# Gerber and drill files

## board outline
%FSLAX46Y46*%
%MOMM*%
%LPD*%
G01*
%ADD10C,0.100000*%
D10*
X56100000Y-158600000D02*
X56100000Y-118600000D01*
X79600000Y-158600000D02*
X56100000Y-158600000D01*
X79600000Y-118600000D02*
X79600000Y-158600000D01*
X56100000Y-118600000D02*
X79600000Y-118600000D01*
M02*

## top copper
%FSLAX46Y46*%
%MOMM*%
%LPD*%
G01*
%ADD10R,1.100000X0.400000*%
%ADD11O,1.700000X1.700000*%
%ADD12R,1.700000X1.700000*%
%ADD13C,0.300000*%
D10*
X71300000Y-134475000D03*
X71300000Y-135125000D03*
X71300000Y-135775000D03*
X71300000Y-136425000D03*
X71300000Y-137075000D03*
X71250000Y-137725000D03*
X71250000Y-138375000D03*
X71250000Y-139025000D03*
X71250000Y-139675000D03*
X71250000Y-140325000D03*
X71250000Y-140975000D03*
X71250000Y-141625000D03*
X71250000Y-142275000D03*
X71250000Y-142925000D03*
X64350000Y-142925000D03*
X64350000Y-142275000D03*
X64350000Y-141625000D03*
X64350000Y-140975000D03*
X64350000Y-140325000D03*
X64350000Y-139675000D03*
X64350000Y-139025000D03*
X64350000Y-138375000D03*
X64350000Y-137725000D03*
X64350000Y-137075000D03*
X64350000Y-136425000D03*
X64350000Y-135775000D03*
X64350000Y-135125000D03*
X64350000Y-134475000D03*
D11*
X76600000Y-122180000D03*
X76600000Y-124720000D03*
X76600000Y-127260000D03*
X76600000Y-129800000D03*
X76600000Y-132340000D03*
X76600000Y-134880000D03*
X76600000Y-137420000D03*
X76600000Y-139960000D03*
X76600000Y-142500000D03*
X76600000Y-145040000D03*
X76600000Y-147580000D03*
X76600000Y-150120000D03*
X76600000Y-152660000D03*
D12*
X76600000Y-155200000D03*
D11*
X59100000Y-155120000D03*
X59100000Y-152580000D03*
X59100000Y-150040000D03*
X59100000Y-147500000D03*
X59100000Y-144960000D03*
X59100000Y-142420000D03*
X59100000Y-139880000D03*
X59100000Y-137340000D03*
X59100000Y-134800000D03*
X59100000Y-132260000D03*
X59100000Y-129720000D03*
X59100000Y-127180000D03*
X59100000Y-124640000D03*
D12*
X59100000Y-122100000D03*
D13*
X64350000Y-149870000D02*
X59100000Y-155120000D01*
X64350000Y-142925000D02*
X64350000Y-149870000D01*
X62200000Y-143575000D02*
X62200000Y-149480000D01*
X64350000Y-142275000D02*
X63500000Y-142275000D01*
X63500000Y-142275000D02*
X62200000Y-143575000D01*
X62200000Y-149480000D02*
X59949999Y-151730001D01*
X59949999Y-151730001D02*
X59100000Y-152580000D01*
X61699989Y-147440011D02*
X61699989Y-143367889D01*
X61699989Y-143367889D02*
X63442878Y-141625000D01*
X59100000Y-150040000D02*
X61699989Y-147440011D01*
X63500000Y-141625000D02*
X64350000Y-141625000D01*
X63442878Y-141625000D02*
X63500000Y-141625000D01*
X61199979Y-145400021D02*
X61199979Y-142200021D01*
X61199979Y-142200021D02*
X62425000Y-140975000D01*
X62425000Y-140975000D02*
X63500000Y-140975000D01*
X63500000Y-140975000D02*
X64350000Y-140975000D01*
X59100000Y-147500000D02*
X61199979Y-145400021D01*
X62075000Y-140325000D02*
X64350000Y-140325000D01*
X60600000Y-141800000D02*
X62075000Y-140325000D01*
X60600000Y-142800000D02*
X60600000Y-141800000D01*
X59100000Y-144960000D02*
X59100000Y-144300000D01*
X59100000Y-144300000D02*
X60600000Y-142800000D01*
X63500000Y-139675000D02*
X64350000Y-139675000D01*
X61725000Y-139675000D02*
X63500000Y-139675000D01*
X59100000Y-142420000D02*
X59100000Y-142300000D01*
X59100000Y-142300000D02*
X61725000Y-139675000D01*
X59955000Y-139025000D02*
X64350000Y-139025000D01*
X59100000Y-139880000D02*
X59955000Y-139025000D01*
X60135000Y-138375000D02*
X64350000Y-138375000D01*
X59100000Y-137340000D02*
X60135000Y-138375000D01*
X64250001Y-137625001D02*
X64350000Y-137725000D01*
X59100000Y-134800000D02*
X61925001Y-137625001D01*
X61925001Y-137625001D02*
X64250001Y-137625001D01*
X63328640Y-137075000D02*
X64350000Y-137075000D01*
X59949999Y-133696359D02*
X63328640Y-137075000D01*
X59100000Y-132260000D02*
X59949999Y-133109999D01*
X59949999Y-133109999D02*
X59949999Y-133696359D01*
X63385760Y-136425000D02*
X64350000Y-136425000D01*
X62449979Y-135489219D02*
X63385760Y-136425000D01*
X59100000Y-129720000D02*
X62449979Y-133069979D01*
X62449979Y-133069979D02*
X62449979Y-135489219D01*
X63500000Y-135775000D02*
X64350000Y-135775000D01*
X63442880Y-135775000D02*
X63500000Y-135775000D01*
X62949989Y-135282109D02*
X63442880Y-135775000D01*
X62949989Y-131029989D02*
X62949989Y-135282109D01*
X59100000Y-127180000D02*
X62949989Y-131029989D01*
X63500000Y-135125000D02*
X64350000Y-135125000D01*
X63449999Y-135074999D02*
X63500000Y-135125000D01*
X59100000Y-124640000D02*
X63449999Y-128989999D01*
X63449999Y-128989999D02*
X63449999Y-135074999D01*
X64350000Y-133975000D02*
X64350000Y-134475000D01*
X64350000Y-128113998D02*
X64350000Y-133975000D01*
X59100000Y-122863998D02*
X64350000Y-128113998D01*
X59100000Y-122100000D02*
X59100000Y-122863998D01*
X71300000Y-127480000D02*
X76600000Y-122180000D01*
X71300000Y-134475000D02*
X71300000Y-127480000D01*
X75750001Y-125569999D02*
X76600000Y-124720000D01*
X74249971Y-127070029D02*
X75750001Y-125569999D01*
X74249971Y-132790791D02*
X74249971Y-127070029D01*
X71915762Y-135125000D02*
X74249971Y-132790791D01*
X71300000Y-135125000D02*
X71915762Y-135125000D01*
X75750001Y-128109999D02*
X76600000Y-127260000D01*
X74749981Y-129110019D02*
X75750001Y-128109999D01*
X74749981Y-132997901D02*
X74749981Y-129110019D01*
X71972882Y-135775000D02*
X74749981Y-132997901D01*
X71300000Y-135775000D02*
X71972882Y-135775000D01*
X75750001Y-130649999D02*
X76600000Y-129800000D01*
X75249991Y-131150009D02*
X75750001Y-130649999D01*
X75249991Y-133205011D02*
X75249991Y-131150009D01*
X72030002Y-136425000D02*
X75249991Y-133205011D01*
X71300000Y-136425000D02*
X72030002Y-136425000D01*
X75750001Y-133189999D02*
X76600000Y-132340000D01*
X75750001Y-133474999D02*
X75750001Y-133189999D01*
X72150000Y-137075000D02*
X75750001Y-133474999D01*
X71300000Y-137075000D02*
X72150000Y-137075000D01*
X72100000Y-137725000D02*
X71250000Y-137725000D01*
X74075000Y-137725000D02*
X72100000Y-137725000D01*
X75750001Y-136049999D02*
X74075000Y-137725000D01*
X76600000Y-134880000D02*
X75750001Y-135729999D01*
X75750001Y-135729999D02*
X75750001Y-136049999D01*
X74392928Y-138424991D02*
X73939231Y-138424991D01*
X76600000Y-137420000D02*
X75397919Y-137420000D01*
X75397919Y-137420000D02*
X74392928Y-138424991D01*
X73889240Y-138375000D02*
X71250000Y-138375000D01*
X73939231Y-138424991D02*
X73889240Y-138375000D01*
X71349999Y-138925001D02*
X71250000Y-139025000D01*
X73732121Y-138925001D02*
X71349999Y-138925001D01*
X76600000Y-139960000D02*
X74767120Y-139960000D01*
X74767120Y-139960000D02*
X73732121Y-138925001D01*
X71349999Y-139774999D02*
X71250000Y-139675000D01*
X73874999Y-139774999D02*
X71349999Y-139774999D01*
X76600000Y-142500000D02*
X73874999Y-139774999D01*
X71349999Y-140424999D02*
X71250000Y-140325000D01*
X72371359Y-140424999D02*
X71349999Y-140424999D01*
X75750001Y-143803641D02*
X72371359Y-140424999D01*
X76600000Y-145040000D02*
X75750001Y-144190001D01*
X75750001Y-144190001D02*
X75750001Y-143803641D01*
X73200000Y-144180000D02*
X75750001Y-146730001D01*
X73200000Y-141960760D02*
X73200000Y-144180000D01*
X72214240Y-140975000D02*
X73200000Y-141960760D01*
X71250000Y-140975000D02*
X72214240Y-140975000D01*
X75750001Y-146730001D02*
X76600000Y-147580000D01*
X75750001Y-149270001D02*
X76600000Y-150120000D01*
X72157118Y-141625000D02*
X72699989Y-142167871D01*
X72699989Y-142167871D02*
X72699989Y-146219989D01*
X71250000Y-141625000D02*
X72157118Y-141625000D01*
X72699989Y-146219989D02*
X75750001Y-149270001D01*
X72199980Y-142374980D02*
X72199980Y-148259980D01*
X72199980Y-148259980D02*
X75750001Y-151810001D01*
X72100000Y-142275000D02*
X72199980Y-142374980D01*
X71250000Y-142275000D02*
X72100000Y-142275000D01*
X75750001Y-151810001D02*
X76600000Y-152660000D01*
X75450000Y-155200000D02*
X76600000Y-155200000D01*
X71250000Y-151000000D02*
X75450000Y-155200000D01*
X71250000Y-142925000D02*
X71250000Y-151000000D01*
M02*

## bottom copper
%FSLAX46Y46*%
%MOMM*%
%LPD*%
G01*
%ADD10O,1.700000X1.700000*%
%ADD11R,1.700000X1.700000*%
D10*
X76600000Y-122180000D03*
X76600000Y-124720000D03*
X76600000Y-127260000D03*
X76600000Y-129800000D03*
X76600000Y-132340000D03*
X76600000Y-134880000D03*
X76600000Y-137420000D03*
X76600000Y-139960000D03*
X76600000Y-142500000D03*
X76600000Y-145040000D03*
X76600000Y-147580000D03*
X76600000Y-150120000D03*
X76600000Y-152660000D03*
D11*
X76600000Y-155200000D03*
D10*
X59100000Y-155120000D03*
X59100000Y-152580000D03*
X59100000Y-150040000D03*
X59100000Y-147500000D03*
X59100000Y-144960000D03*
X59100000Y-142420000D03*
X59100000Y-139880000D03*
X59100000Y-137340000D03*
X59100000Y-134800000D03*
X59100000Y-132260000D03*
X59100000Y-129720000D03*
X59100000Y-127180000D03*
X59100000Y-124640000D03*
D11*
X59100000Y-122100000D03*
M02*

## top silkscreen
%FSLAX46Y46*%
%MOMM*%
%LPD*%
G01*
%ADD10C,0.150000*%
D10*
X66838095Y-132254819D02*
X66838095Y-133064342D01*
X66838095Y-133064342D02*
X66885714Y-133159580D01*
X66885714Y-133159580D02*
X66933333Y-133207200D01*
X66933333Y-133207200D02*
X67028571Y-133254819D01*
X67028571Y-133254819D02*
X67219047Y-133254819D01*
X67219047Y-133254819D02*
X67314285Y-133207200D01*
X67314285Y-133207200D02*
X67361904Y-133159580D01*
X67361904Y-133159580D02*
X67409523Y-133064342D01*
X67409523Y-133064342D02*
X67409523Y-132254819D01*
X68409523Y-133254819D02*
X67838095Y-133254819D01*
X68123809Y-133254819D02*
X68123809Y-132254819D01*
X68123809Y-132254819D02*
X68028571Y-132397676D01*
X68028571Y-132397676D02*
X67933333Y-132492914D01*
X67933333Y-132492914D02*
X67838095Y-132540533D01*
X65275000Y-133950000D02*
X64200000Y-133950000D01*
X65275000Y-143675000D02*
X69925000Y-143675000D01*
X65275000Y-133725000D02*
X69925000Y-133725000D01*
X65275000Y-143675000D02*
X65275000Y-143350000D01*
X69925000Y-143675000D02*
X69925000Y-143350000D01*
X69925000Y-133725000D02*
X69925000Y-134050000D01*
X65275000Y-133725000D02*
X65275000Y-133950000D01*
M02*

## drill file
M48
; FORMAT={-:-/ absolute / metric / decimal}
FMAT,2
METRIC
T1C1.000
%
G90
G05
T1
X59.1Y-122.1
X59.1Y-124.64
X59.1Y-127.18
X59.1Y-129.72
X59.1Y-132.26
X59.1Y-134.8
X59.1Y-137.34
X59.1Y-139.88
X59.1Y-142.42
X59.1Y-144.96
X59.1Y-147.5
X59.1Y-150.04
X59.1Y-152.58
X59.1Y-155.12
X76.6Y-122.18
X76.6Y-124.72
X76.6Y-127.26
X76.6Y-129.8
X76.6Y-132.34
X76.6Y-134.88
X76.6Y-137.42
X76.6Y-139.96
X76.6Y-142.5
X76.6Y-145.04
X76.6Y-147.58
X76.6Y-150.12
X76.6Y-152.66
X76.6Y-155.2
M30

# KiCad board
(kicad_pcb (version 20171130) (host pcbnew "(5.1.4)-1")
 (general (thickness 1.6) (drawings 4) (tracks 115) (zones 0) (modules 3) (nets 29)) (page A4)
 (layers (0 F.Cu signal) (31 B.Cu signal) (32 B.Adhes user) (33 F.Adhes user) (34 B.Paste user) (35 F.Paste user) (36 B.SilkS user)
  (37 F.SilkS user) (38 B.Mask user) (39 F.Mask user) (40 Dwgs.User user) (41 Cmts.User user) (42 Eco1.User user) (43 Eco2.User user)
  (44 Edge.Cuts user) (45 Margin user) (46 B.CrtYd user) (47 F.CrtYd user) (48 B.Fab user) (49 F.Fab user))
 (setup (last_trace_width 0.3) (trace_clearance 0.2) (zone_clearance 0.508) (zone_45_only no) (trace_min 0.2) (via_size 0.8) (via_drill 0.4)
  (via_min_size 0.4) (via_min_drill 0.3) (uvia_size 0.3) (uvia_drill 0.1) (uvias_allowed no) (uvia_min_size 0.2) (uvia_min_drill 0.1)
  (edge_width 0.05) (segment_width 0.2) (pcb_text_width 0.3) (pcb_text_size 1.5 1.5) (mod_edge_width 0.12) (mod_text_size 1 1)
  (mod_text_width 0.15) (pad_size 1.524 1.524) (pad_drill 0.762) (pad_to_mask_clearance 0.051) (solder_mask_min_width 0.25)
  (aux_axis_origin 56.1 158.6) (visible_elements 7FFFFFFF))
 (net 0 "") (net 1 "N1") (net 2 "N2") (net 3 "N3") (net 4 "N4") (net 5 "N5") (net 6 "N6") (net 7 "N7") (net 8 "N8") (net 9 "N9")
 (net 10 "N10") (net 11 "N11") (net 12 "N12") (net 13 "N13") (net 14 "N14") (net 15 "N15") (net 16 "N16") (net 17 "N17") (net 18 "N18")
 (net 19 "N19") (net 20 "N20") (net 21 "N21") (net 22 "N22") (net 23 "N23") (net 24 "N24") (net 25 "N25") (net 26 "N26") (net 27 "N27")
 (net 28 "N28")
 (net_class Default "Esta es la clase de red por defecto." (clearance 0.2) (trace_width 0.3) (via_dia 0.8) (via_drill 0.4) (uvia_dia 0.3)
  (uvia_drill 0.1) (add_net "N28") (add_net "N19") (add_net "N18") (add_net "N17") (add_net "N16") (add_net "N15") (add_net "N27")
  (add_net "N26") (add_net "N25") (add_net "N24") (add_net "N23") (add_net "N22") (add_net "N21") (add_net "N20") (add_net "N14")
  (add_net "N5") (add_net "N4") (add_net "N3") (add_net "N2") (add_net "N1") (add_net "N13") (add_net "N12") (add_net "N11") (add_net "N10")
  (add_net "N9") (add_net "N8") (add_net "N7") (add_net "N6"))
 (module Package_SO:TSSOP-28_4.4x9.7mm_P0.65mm (layer F.Cu) (at 67.6 138.7)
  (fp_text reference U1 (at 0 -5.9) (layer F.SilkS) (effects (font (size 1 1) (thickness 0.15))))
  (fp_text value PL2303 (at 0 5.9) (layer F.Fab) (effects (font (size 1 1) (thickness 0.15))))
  (fp_line (start -2.325 -4.75) (end -3.4 -4.75) (layer F.SilkS) (width 0.15))
  (fp_line (start -2.325 4.975) (end 2.325 4.975) (layer F.SilkS) (width 0.15))
  (fp_line (start -2.325 -4.975) (end 2.325 -4.975) (layer F.SilkS) (width 0.15))
  (fp_line (start -2.325 4.975) (end -2.325 4.65) (layer F.SilkS) (width 0.15))
  (fp_line (start 2.325 4.975) (end 2.325 4.65) (layer F.SilkS) (width 0.15))
  (fp_line (start 2.325 -4.975) (end 2.325 -4.65) (layer F.SilkS) (width 0.15))
  (fp_line (start -2.325 -4.975) (end -2.325 -4.75) (layer F.SilkS) (width 0.15))
  (pad 28 smd rect (at 3.7 -4.225) (size 1.1 0.4) (layers F.Cu F.Paste F.Mask) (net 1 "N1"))
  (pad 27 smd rect (at 3.7 -3.575) (size 1.1 0.4) (layers F.Cu F.Paste F.Mask) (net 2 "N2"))
  (pad 26 smd rect (at 3.7 -2.925) (size 1.1 0.4) (layers F.Cu F.Paste F.Mask) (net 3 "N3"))
  (pad 25 smd rect (at 3.7 -2.275) (size 1.1 0.4) (layers F.Cu F.Paste F.Mask) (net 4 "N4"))
  (pad 24 smd rect (at 3.7 -1.625) (size 1.1 0.4) (layers F.Cu F.Paste F.Mask) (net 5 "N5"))
  (pad 23 smd rect (at 3.65 -0.975) (size 1.1 0.4) (layers F.Cu F.Paste F.Mask) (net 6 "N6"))
  (pad 22 smd rect (at 3.65 -0.325) (size 1.1 0.4) (layers F.Cu F.Paste F.Mask) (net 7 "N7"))
  (pad 21 smd rect (at 3.65 0.325) (size 1.1 0.4) (layers F.Cu F.Paste F.Mask) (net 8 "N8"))
  (pad 20 smd rect (at 3.65 0.975) (size 1.1 0.4) (layers F.Cu F.Paste F.Mask) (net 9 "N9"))
  (pad 19 smd rect (at 3.65 1.625) (size 1.1 0.4) (layers F.Cu F.Paste F.Mask) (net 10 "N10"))
  (pad 18 smd rect (at 3.65 2.275) (size 1.1 0.4) (layers F.Cu F.Paste F.Mask) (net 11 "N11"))
  (pad 17 smd rect (at 3.65 2.925) (size 1.1 0.4) (layers F.Cu F.Paste F.Mask) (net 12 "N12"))
  (pad 16 smd rect (at 3.65 3.575) (size 1.1 0.4) (layers F.Cu F.Paste F.Mask) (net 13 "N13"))
  (pad 15 smd rect (at 3.65 4.225) (size 1.1 0.4) (layers F.Cu F.Paste F.Mask) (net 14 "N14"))
  (pad 14 smd rect (at -3.25 4.225) (size 1.1 0.4) (layers F.Cu F.Paste F.Mask) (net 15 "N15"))
  (pad 13 smd rect (at -3.25 3.575) (size 1.1 0.4) (layers F.Cu F.Paste F.Mask) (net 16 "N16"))
  (pad 12 smd rect (at -3.25 2.925) (size 1.1 0.4) (layers F.Cu F.Paste F.Mask) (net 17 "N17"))
  (pad 11 smd rect (at -3.25 2.275) (size 1.1 0.4) (layers F.Cu F.Paste F.Mask) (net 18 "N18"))
  (pad 10 smd rect (at -3.25 1.625) (size 1.1 0.4) (layers F.Cu F.Paste F.Mask) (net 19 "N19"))
  (pad 9 smd rect (at -3.25 0.975) (size 1.1 0.4) (layers F.Cu F.Paste F.Mask) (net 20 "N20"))
  (pad 8 smd rect (at -3.25 0.325) (size 1.1 0.4) (layers F.Cu F.Paste F.Mask) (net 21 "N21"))
  (pad 7 smd rect (at -3.25 -0.325) (size 1.1 0.4) (layers F.Cu F.Paste F.Mask) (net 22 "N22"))
  (pad 6 smd rect (at -3.25 -0.975) (size 1.1 0.4) (layers F.Cu F.Paste F.Mask) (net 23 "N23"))
  (pad 5 smd rect (at -3.25 -1.625) (size 1.1 0.4) (layers F.Cu F.Paste F.Mask) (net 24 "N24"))
  (pad 4 smd rect (at -3.25 -2.275) (size 1.1 0.4) (layers F.Cu F.Paste F.Mask) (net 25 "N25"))
  (pad 3 smd rect (at -3.25 -2.925) (size 1.1 0.4) (layers F.Cu F.Paste F.Mask) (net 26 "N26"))
  (pad 2 smd rect (at -3.25 -3.575) (size 1.1 0.4) (layers F.Cu F.Paste F.Mask) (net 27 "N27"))
  (pad 1 smd rect (at -3.25 -4.225) (size 1.1 0.4) (layers F.Cu F.Paste F.Mask) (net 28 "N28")))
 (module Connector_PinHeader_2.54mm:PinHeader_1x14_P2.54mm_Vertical (layer B.Cu) (at 76.6 155.2)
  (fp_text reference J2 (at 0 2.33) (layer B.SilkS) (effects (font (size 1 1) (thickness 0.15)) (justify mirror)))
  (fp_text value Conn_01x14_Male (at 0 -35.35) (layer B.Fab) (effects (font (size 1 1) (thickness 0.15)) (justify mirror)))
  (pad 14 thru_hole oval (at 0 -33.02) (size 1.7 1.7) (drill 1) (layers *.Cu *.Mask) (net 1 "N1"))
  (pad 13 thru_hole oval (at 0 -30.48) (size 1.7 1.7) (drill 1) (layers *.Cu *.Mask) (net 2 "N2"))
  (pad 12 thru_hole oval (at 0 -27.94) (size 1.7 1.7) (drill 1) (layers *.Cu *.Mask) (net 3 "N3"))
  (pad 11 thru_hole oval (at 0 -25.4) (size 1.7 1.7) (drill 1) (layers *.Cu *.Mask) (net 4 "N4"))
  (pad 10 thru_hole oval (at 0 -22.86) (size 1.7 1.7) (drill 1) (layers *.Cu *.Mask) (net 5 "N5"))
  (pad 9 thru_hole oval (at 0 -20.32) (size 1.7 1.7) (drill 1) (layers *.Cu *.Mask) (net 6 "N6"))
  (pad 8 thru_hole oval (at 0 -17.78) (size 1.7 1.7) (drill 1) (layers *.Cu *.Mask) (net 7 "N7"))
  (pad 7 thru_hole oval (at 0 -15.24) (size 1.7 1.7) (drill 1) (layers *.Cu *.Mask) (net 8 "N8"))
  (pad 6 thru_hole oval (at 0 -12.7) (size 1.7 1.7) (drill 1) (layers *.Cu *.Mask) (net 9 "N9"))
  (pad 5 thru_hole oval (at 0 -10.16) (size 1.7 1.7) (drill 1) (layers *.Cu *.Mask) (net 10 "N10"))
  (pad 4 thru_hole oval (at 0 -7.62) (size 1.7 1.7) (drill 1) (layers *.Cu *.Mask) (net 11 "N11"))
  (pad 3 thru_hole oval (at 0 -5.08) (size 1.7 1.7) (drill 1) (layers *.Cu *.Mask) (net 12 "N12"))
  (pad 2 thru_hole oval (at 0 -2.54) (size 1.7 1.7) (drill 1) (layers *.Cu *.Mask) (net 13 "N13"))
  (pad 1 thru_hole rect (at 0 0) (size 1.7 1.7) (drill 1) (layers *.Cu *.Mask) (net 14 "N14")))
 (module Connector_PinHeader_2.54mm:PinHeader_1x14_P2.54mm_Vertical (layer B.Cu) (at 59.1 122.1 180)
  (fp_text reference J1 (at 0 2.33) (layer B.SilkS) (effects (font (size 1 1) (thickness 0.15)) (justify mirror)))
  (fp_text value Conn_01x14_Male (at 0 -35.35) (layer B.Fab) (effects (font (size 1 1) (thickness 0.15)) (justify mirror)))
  (pad 14 thru_hole oval (at 0 -33.02 180) (size 1.7 1.7) (drill 1) (layers *.Cu *.Mask) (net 15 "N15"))
  (pad 13 thru_hole oval (at 0 -30.48 180) (size 1.7 1.7) (drill 1) (layers *.Cu *.Mask) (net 16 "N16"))
  (pad 12 thru_hole oval (at 0 -27.94 180) (size 1.7 1.7) (drill 1) (layers *.Cu *.Mask) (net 17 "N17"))
  (pad 11 thru_hole oval (at 0 -25.4 180) (size 1.7 1.7) (drill 1) (layers *.Cu *.Mask) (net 18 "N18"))
  (pad 10 thru_hole oval (at 0 -22.86 180) (size 1.7 1.7) (drill 1) (layers *.Cu *.Mask) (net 19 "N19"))
  (pad 9 thru_hole oval (at 0 -20.32 180) (size 1.7 1.7) (drill 1) (layers *.Cu *.Mask) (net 20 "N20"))
  (pad 8 thru_hole oval (at 0 -17.78 180) (size 1.7 1.7) (drill 1) (layers *.Cu *.Mask) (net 21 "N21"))
  (pad 7 thru_hole oval (at 0 -15.24 180) (size 1.7 1.7) (drill 1) (layers *.Cu *.Mask) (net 22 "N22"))
  (pad 6 thru_hole oval (at 0 -12.7 180) (size 1.7 1.7) (drill 1) (layers *.Cu *.Mask) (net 23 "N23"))
  (pad 5 thru_hole oval (at 0 -10.16 180) (size 1.7 1.7) (drill 1) (layers *.Cu *.Mask) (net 24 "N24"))
  (pad 4 thru_hole oval (at 0 -7.62 180) (size 1.7 1.7) (drill 1) (layers *.Cu *.Mask) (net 25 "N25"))
  (pad 3 thru_hole oval (at 0 -5.08 180) (size 1.7 1.7) (drill 1) (layers *.Cu *.Mask) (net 26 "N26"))
  (pad 2 thru_hole oval (at 0 -2.54 180) (size 1.7 1.7) (drill 1) (layers *.Cu *.Mask) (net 27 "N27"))
  (pad 1 thru_hole rect (at 0 0 180) (size 1.7 1.7) (drill 1) (layers *.Cu *.Mask) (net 28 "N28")))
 (gr_line (start 56.1 158.6) (end 56.1 118.6) (layer Edge.Cuts) (width 0.1))
 (gr_line (start 79.6 158.6) (end 56.1 158.6) (layer Edge.Cuts) (width 0.1))
 (gr_line (start 79.6 118.6) (end 79.6 158.6) (layer Edge.Cuts) (width 0.1))
 (gr_line (start 56.1 118.6) (end 79.6 118.6) (layer Edge.Cuts) (width 0.1))
 (segment (start 64.35 149.87) (end 59.1 155.12) (width 0.3) (layer F.Cu) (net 15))
 (segment (start 64.35 142.925) (end 64.35 149.87) (width 0.3) (layer F.Cu) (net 15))
 (segment (start 62.2 143.575) (end 62.2 149.48) (width 0.3) (layer F.Cu) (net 16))
 (segment (start 64.35 142.275) (end 63.5 142.275) (width 0.3) (layer F.Cu) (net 16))
 (segment (start 63.5 142.275) (end 62.2 143.575) (width 0.3) (layer F.Cu) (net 16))
 (segment (start 62.2 149.48) (end 59.949999 151.730001) (width 0.3) (layer F.Cu) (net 16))
 (segment (start 59.949999 151.730001) (end 59.1 152.58) (width 0.3) (layer F.Cu) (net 16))
 (segment (start 61.699989 147.440011) (end 61.699989 143.367889) (width 0.3) (layer F.Cu) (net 17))
 (segment (start 61.699989 143.367889) (end 63.442878 141.625) (width 0.3) (layer F.Cu) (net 17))
 (segment (start 59.1 150.04) (end 61.699989 147.440011) (width 0.3) (layer F.Cu) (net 17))
 (segment (start 63.5 141.625) (end 64.35 141.625) (width 0.3) (layer F.Cu) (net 17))
 (segment (start 63.442878 141.625) (end 63.5 141.625) (width 0.3) (layer F.Cu) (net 17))
 (segment (start 61.199979 145.400021) (end 61.199979 142.200021) (width 0.3) (layer F.Cu) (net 18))
 (segment (start 61.199979 142.200021) (end 62.425 140.975) (width 0.3) (layer F.Cu) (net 18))
 (segment (start 62.425 140.975) (end 63.5 140.975) (width 0.3) (layer F.Cu) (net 18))
 (segment (start 63.5 140.975) (end 64.35 140.975) (width 0.3) (layer F.Cu) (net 18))
 (segment (start 59.1 147.5) (end 61.199979 145.400021) (width 0.3) (layer F.Cu) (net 18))
 (segment (start 62.075 140.325) (end 64.35 140.325) (width 0.3) (layer F.Cu) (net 19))
 (segment (start 60.6 141.8) (end 62.075 140.325) (width 0.3) (layer F.Cu) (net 19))
 (segment (start 60.6 142.8) (end 60.6 141.8) (width 0.3) (layer F.Cu) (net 19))
 (segment (start 59.1 144.96) (end 59.1 144.3) (width 0.3) (layer F.Cu) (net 19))
 (segment (start 59.1 144.3) (end 60.6 142.8) (width 0.3) (layer F.Cu) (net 19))
 (segment (start 63.5 139.675) (end 64.35 139.675) (width 0.3) (layer F.Cu) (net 20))
 (segment (start 61.725 139.675) (end 63.5 139.675) (width 0.3) (layer F.Cu) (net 20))
 (segment (start 59.1 142.42) (end 59.1 142.3) (width 0.3) (layer F.Cu) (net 20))
 (segment (start 59.1 142.3) (end 61.725 139.675) (width 0.3) (layer F.Cu) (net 20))
 (segment (start 59.955 139.025) (end 64.35 139.025) (width 0.3) (layer F.Cu) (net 21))
 (segment (start 59.1 139.88) (end 59.955 139.025) (width 0.3) (layer F.Cu) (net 21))
 (segment (start 60.135 138.375) (end 64.35 138.375) (width 0.3) (layer F.Cu) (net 22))
 (segment (start 59.1 137.34) (end 60.135 138.375) (width 0.3) (layer F.Cu) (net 22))
 (segment (start 64.250001 137.625001) (end 64.35 137.725) (width 0.3) (layer F.Cu) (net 23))
 (segment (start 59.1 134.8) (end 61.925001 137.625001) (width 0.3) (layer F.Cu) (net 23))
 (segment (start 61.925001 137.625001) (end 64.250001 137.625001) (width 0.3) (layer F.Cu) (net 23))
 (segment (start 63.32864 137.075) (end 64.35 137.075) (width 0.3) (layer F.Cu) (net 24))
 (segment (start 59.949999 133.696359) (end 63.32864 137.075) (width 0.3) (layer F.Cu) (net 24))
 (segment (start 59.1 132.26) (end 59.949999 133.109999) (width 0.3) (layer F.Cu) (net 24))
 (segment (start 59.949999 133.109999) (end 59.949999 133.696359) (width 0.3) (layer F.Cu) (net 24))
 (segment (start 63.38576 136.425) (end 64.35 136.425) (width 0.3) (layer F.Cu) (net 25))
 (segment (start 62.449979 135.489219) (end 63.38576 136.425) (width 0.3) (layer F.Cu) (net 25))
 (segment (start 59.1 129.72) (end 62.449979 133.069979) (width 0.3) (layer F.Cu) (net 25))
 (segment (start 62.449979 133.069979) (end 62.449979 135.489219) (width 0.3) (layer F.Cu) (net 25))
 (segment (start 63.5 135.775) (end 64.35 135.775) (width 0.3) (layer F.Cu) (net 26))
 (segment (start 63.44288 135.775) (end 63.5 135.775) (width 0.3) (layer F.Cu) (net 26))
 (segment (start 62.949989 135.282109) (end 63.44288 135.775) (width 0.3) (layer F.Cu) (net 26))
 (segment (start 62.949989 131.029989) (end 62.949989 135.282109) (width 0.3) (layer F.Cu) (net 26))
 (segment (start 59.1 127.18) (end 62.949989 131.029989) (width 0.3) (layer F.Cu) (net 26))
 (segment (start 63.5 135.125) (end 64.35 135.125) (width 0.3) (layer F.Cu) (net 27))
 (segment (start 63.449999 135.074999) (end 63.5 135.125) (width 0.3) (layer F.Cu) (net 27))
 (segment (start 59.1 124.64) (end 63.449999 128.989999) (width 0.3) (layer F.Cu) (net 27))
 (segment (start 63.449999 128.989999) (end 63.449999 135.074999) (width 0.3) (layer F.Cu) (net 27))
 (segment (start 64.35 133.975) (end 64.35 134.475) (width 0.3) (layer F.Cu) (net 28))
 (segment (start 64.35 128.113998) (end 64.35 133.975) (width 0.3) (layer F.Cu) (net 28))
 (segment (start 59.1 122.863998) (end 64.35 128.113998) (width 0.3) (layer F.Cu) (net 28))
 (segment (start 59.1 122.1) (end 59.1 122.863998) (width 0.3) (layer F.Cu) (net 28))
 (segment (start 71.3 127.48) (end 76.6 122.18) (width 0.3) (layer F.Cu) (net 1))
 (segment (start 71.3 134.475) (end 71.3 127.48) (width 0.3) (layer F.Cu) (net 1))
 (segment (start 75.750001 125.569999) (end 76.6 124.72) (width 0.3) (layer F.Cu) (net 2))
 (segment (start 74.249971 127.070029) (end 75.750001 125.569999) (width 0.3) (layer F.Cu) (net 2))
 (segment (start 74.249971 132.790791) (end 74.249971 127.070029) (width 0.3) (layer F.Cu) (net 2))
 (segment (start 71.915762 135.125) (end 74.249971 132.790791) (width 0.3) (layer F.Cu) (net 2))
 (segment (start 71.3 135.125) (end 71.915762 135.125) (width 0.3) (layer F.Cu) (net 2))
 (segment (start 75.750001 128.109999) (end 76.6 127.26) (width 0.3) (layer F.Cu) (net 3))
 (segment (start 74.749981 129.110019) (end 75.750001 128.109999) (width 0.3) (layer F.Cu) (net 3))
 (segment (start 74.749981 132.997901) (end 74.749981 129.110019) (width 0.3) (layer F.Cu) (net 3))
 (segment (start 71.972882 135.775) (end 74.749981 132.997901) (width 0.3) (layer F.Cu) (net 3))
 (segment (start 71.3 135.775) (end 71.972882 135.775) (width 0.3) (layer F.Cu) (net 3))
 (segment (start 75.750001 130.649999) (end 76.6 129.8) (width 0.3) (layer F.Cu) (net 4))
 (segment (start 75.249991 131.150009) (end 75.750001 130.649999) (width 0.3) (layer F.Cu) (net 4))
 (segment (start 75.249991 133.205011) (end 75.249991 131.150009) (width 0.3) (layer F.Cu) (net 4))
 (segment (start 72.030002 136.425) (end 75.249991 133.205011) (width 0.3) (layer F.Cu) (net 4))
 (segment (start 71.3 136.425) (end 72.030002 136.425) (width 0.3) (layer F.Cu) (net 4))
 (segment (start 75.750001 133.189999) (end 76.6 132.34) (width 0.3) (layer F.Cu) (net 5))
 (segment (start 75.750001 133.474999) (end 75.750001 133.189999) (width 0.3) (layer F.Cu) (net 5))
 (segment (start 72.15 137.075) (end 75.750001 133.474999) (width 0.3) (layer F.Cu) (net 5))
 (segment (start 71.3 137.075) (end 72.15 137.075) (width 0.3) (layer F.Cu) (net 5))
 (segment (start 72.1 137.725) (end 71.25 137.725) (width 0.3) (layer F.Cu) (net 6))
 (segment (start 74.075 137.725) (end 72.1 137.725) (width 0.3) (layer F.Cu) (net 6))
 (segment (start 75.750001 136.049999) (end 74.075 137.725) (width 0.3) (layer F.Cu) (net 6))
 (segment (start 76.6 134.88) (end 75.750001 135.729999) (width 0.3) (layer F.Cu) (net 6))
 (segment (start 75.750001 135.729999) (end 75.750001 136.049999) (width 0.3) (layer F.Cu) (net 6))
 (segment (start 74.392928 138.424991) (end 73.939231 138.424991) (width 0.3) (layer F.Cu) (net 7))
 (segment (start 76.6 137.42) (end 75.397919 137.42) (width 0.3) (layer F.Cu) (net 7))
 (segment (start 75.397919 137.42) (end 74.392928 138.424991) (width 0.3) (layer F.Cu) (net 7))
 (segment (start 73.88924 138.375) (end 71.25 138.375) (width 0.3) (layer F.Cu) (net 7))
 (segment (start 73.939231 138.424991) (end 73.88924 138.375) (width 0.3) (layer F.Cu) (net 7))
 (segment (start 71.349999 138.925001) (end 71.25 139.025) (width 0.3) (layer F.Cu) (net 8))
 (segment (start 73.732121 138.925001) (end 71.349999 138.925001) (width 0.3) (layer F.Cu) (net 8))
 (segment (start 76.6 139.96) (end 74.76712 139.96) (width 0.3) (layer F.Cu) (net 8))
 (segment (start 74.76712 139.96) (end 73.732121 138.925001) (width 0.3) (layer F.Cu) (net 8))
 (segment (start 71.349999 139.774999) (end 71.25 139.675) (width 0.3) (layer F.Cu) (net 9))
 (segment (start 73.874999 139.774999) (end 71.349999 139.774999) (width 0.3) (layer F.Cu) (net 9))
 (segment (start 76.6 142.5) (end 73.874999 139.774999) (width 0.3) (layer F.Cu) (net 9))
 (segment (start 71.349999 140.424999) (end 71.25 140.325) (width 0.3) (layer F.Cu) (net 10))
 (segment (start 72.371359 140.424999) (end 71.349999 140.424999) (width 0.3) (layer F.Cu) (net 10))
 (segment (start 75.750001 143.803641) (end 72.371359 140.424999) (width 0.3) (layer F.Cu) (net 10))
 (segment (start 76.6 145.04) (end 75.750001 144.190001) (width 0.3) (layer F.Cu) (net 10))
 (segment (start 75.750001 144.190001) (end 75.750001 143.803641) (width 0.3) (layer F.Cu) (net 10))
 (segment (start 73.2 144.18) (end 75.750001 146.730001) (width 0.3) (layer F.Cu) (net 11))
 (segment (start 73.2 141.96076) (end 73.2 144.18) (width 0.3) (layer F.Cu) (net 11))
 (segment (start 72.21424 140.975) (end 73.2 141.96076) (width 0.3) (layer F.Cu) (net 11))
 (segment (start 71.25 140.975) (end 72.21424 140.975) (width 0.3) (layer F.Cu) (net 11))
 (segment (start 75.750001 146.730001) (end 76.6 147.58) (width 0.3) (layer F.Cu) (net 11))
 (segment (start 75.750001 149.270001) (end 76.6 150.12) (width 0.3) (layer F.Cu) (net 12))
 (segment (start 72.157118 141.625) (end 72.699989 142.167871) (width 0.3) (layer F.Cu) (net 12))
 (segment (start 72.699989 142.167871) (end 72.699989 146.219989) (width 0.3) (layer F.Cu) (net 12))
 (segment (start 71.25 141.625) (end 72.157118 141.625) (width 0.3) (layer F.Cu) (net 12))
 (segment (start 72.699989 146.219989) (end 75.750001 149.270001) (width 0.3) (layer F.Cu) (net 12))
 (segment (start 72.19998 142.37498) (end 72.19998 148.25998) (width 0.3) (layer F.Cu) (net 13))
 (segment (start 72.19998 148.25998) (end 75.750001 151.810001) (width 0.3) (layer F.Cu) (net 13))
 (segment (start 72.1 142.275) (end 72.19998 142.37498) (width 0.3) (layer F.Cu) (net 13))
 (segment (start 71.25 142.275) (end 72.1 142.275) (width 0.3) (layer F.Cu) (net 13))
 (segment (start 75.750001 151.810001) (end 76.6 152.66) (width 0.3) (layer F.Cu) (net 13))
 (segment (start 75.45 155.2) (end 76.6 155.2) (width 0.3) (layer F.Cu) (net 14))
 (segment (start 71.25 151) (end 75.45 155.2) (width 0.3) (layer F.Cu) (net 14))
 (segment (start 71.25 142.925) (end 71.25 151) (width 0.3) (layer F.Cu) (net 14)))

